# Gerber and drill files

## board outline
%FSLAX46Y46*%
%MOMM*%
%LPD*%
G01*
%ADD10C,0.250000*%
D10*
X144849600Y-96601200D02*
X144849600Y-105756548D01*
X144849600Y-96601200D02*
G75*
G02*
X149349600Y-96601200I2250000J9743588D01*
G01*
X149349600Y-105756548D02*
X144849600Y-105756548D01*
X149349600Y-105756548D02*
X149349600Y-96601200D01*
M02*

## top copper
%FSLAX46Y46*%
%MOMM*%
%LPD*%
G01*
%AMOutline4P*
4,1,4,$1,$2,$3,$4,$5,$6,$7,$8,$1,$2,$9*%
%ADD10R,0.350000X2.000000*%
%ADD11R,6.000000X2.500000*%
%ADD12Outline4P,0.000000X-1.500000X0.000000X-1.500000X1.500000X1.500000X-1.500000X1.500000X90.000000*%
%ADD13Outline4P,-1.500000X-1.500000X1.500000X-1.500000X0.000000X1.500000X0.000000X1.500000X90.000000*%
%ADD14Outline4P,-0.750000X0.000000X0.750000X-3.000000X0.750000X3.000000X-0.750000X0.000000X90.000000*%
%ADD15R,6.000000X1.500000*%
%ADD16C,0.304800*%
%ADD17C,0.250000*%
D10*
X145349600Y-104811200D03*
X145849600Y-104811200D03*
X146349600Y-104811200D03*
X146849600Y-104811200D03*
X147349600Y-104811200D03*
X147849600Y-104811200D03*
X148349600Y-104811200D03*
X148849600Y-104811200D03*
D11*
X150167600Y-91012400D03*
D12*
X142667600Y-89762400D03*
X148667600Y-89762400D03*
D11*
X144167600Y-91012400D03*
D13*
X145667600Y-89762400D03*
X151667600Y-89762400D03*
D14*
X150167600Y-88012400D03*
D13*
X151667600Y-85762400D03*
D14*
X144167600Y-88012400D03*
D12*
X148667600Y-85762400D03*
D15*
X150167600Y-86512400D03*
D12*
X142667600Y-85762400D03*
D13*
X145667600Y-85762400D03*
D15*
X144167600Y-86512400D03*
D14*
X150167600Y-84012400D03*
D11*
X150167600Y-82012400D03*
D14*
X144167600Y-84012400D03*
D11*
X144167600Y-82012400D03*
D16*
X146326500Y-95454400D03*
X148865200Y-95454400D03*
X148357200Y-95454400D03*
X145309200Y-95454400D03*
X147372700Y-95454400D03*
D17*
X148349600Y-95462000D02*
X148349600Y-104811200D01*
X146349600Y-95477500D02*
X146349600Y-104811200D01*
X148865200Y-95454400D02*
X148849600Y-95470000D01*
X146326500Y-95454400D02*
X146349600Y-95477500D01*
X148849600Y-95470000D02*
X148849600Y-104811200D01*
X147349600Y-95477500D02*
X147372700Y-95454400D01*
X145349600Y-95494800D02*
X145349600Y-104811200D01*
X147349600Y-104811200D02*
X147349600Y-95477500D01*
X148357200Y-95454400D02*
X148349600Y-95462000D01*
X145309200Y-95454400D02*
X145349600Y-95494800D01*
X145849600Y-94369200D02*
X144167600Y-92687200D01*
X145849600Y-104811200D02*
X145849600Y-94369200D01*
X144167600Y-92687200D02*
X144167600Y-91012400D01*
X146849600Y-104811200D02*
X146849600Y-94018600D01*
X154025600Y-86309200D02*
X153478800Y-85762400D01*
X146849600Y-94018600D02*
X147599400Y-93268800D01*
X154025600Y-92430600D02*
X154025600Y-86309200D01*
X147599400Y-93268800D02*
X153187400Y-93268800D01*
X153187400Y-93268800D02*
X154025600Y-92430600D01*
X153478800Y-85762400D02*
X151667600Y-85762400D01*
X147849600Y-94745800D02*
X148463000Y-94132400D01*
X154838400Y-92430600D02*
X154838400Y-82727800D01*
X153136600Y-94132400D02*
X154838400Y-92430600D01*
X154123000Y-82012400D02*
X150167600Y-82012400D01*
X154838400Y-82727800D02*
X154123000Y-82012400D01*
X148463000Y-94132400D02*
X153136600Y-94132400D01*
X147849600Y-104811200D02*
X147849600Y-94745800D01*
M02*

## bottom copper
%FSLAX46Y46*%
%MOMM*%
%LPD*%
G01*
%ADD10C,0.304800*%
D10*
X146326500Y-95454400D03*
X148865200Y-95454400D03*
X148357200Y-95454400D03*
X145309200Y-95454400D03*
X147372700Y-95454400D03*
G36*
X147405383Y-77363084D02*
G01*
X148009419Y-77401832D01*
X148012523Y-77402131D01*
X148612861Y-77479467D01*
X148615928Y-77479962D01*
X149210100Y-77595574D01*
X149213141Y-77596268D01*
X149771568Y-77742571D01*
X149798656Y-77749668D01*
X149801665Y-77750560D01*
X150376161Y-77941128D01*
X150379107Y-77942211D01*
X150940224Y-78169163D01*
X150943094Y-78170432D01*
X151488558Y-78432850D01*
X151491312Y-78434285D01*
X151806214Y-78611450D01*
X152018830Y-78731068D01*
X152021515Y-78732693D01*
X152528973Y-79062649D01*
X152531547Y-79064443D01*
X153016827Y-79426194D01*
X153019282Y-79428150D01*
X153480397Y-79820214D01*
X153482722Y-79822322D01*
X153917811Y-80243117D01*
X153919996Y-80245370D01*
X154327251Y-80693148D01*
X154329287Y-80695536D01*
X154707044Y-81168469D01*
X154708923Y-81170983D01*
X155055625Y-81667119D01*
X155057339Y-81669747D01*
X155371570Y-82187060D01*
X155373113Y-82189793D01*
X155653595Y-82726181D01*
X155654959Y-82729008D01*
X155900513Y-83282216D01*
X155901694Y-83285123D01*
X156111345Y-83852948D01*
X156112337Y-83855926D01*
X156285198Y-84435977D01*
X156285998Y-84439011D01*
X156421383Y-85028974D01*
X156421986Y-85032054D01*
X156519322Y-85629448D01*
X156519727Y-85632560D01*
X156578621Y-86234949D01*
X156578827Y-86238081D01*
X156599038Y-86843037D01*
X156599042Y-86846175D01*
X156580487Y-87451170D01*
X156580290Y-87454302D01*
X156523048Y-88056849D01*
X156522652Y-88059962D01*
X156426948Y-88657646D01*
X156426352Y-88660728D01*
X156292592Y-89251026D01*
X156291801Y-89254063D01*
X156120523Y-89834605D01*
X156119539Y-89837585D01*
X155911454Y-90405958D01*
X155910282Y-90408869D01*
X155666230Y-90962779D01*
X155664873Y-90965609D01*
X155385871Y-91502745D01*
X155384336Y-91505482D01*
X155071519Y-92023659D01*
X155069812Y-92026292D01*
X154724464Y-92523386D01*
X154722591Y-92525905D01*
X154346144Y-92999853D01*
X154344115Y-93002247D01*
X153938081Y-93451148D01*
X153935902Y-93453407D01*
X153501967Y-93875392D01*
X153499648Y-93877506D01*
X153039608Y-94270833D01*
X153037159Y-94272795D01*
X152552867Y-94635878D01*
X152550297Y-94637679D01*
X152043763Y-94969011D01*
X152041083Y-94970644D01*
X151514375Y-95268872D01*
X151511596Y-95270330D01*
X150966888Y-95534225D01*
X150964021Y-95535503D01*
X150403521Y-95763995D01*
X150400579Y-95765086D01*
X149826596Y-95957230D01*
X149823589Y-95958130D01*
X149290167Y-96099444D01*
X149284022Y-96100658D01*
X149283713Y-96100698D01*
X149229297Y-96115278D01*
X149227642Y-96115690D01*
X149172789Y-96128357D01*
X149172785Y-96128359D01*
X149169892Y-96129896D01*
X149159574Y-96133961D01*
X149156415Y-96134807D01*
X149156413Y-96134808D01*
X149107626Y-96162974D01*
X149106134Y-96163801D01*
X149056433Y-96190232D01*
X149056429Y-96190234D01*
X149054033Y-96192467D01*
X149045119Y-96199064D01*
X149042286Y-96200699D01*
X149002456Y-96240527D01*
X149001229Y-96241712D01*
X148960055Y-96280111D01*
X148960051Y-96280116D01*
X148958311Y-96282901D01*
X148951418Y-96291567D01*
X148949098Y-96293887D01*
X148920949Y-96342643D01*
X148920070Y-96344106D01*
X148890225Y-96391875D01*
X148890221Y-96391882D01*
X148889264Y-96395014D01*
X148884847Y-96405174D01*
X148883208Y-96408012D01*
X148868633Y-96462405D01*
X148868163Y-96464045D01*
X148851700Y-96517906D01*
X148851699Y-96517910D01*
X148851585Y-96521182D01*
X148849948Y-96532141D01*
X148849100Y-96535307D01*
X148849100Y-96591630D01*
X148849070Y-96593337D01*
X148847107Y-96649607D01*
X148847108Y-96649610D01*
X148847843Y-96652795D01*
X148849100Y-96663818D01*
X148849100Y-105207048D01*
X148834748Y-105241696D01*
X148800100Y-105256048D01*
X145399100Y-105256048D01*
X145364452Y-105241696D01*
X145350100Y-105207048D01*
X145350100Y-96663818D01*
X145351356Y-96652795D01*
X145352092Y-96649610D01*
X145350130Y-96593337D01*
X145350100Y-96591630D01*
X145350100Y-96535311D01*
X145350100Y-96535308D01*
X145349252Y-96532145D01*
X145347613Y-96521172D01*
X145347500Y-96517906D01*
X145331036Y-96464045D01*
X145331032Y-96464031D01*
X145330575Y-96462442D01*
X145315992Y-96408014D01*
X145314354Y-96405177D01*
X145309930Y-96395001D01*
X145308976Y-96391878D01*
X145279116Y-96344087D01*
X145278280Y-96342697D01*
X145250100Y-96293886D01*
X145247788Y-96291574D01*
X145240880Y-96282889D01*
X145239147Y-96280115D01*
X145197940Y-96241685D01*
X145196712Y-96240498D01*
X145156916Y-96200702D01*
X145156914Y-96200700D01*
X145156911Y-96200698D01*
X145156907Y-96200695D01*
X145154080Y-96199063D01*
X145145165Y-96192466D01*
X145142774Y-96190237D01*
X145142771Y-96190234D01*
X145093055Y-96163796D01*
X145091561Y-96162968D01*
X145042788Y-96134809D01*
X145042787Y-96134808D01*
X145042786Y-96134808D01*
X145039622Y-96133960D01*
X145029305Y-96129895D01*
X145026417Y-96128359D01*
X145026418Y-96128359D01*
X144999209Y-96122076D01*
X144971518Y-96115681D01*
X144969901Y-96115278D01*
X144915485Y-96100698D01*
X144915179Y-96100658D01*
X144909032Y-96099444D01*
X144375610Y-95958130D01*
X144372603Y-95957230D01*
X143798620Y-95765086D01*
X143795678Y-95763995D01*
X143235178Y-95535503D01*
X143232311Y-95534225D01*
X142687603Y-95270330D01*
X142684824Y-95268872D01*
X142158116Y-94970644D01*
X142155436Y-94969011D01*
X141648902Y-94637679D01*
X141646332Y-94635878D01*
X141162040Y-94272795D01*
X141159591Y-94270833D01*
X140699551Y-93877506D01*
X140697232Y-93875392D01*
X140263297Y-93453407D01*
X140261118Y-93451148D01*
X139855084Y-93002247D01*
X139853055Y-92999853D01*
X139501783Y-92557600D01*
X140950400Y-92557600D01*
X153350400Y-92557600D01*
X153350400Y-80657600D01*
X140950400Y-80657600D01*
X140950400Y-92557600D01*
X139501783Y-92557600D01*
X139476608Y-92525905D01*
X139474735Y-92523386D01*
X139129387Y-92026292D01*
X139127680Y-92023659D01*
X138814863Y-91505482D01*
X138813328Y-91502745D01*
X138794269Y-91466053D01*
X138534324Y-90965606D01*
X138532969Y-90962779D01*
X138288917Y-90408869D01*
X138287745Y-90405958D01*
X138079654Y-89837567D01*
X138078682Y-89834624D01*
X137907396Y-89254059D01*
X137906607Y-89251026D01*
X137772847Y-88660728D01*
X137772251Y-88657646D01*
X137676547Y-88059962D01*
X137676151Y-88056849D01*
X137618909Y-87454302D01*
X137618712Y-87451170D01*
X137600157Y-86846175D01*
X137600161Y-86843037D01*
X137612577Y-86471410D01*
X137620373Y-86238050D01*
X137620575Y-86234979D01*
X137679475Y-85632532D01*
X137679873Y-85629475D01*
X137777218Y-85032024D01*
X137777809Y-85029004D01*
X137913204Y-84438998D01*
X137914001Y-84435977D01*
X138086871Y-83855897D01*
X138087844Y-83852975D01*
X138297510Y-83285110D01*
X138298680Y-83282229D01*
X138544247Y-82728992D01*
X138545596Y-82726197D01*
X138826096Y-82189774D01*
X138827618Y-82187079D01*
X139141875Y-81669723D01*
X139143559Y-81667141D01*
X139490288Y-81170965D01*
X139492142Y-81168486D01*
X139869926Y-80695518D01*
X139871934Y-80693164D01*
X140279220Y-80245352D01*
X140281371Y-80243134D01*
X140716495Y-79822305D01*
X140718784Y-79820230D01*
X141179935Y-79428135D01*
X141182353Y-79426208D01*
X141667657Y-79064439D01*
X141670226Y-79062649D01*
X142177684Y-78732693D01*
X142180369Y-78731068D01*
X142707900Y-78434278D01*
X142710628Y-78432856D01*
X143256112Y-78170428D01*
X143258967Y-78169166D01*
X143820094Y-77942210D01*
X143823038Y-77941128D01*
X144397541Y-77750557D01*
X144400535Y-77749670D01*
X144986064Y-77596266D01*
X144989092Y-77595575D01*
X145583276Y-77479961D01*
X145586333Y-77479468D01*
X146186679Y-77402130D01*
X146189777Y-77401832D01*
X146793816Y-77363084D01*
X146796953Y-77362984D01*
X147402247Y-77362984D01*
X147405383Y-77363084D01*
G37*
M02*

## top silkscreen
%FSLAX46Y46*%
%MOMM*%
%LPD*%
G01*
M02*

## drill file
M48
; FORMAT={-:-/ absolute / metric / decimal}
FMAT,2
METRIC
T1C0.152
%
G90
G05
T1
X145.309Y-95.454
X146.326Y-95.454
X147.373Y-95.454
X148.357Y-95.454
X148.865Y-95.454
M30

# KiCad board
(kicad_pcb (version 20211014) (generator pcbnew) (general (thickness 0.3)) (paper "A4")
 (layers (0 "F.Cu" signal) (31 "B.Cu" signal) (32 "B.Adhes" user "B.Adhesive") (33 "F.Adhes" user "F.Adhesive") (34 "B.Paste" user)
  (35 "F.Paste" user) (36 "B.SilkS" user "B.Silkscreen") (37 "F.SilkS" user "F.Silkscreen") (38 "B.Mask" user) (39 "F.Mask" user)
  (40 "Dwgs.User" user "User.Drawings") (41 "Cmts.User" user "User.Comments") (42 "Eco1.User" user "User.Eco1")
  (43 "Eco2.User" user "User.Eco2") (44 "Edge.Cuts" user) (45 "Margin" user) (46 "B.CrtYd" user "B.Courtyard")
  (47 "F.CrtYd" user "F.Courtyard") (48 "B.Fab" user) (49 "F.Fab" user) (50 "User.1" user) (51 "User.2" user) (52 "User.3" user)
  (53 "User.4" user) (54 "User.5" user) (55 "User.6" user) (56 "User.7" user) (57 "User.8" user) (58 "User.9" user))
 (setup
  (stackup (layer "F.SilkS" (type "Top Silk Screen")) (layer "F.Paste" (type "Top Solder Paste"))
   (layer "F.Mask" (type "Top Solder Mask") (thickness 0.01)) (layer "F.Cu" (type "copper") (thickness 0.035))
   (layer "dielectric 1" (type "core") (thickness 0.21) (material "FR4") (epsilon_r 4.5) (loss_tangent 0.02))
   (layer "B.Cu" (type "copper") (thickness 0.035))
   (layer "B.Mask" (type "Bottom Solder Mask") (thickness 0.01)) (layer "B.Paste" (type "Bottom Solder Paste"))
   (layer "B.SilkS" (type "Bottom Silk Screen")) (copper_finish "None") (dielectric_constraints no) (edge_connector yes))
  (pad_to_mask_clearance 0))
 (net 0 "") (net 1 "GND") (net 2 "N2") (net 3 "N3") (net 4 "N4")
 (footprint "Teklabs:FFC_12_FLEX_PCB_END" (layer "F.Cu") (at 148.0996 104.6112)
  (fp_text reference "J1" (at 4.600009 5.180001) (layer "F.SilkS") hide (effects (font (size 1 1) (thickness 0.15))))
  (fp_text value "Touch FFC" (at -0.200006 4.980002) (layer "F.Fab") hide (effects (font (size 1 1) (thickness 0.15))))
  (pad "1" smd rect (at -2.75 0.2 180) (size 0.35 2) (layers "F.Cu" "F.Paste" "F.Mask") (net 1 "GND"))
  (pad "2" smd rect (at -2.25 0.2 180) (size 0.35 2) (layers "F.Cu" "F.Paste" "F.Mask") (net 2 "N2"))
  (pad "3" smd rect (at -1.75 0.2 180) (size 0.35 2) (layers "F.Cu" "F.Paste" "F.Mask") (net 1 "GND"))
  (pad "4" smd rect (at -1.25 0.2 180) (size 0.35 2) (layers "F.Cu" "F.Paste" "F.Mask") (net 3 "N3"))
  (pad "5" smd rect (at -0.75 0.2 180) (size 0.35 2) (layers "F.Cu" "F.Paste" "F.Mask") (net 1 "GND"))
  (pad "6" smd rect (at -0.25 0.2 180) (size 0.35 2) (layers "F.Cu" "F.Paste" "F.Mask") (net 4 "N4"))
  (pad "7" smd rect (at 0.25 0.2 180) (size 0.35 2) (layers "F.Cu" "F.Paste" "F.Mask") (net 1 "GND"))
  (pad "8" smd rect (at 0.75 0.2 180) (size 0.35 2) (layers "F.Cu" "F.Paste" "F.Mask") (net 1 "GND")))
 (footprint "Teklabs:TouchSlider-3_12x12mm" (layer "F.Cu") (at 146.3276 87.3524)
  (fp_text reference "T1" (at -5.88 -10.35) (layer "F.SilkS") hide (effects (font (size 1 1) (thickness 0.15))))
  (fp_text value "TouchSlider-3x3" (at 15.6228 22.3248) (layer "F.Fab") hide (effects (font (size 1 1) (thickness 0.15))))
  (pad "1" smd rect (at 3.84 3.66 90) (size 2.5 6) (layers "F.Cu" "F.Mask") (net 2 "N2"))
  (pad "1" smd trapezoid (at -3.66 2.41 90) (size 1.5 3) (rect_delta 0 -1.5) (layers "F.Cu" "F.Mask") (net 2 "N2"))
  (pad "1" smd trapezoid (at 2.34 2.41 90) (size 1.5 3) (rect_delta 0 -1.5) (layers "F.Cu" "F.Mask") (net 2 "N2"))
  (pad "1" smd rect (at -2.16 3.66 90) (size 2.5 6) (layers "F.Cu" "F.Mask") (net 2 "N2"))
  (pad "1" smd trapezoid (at -0.66 2.41 90) (size 1.5 3) (rect_delta 0 1.5) (layers "F.Cu" "F.Mask") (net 2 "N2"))
  (pad "1" smd trapezoid (at 5.34 2.41 90) (size 1.5 3) (rect_delta 0 1.5) (layers "F.Cu" "F.Mask") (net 2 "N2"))
  (pad "2" smd trapezoid (at 3.84 0.66 90) (size 1.5 3) (rect_delta -3 0) (layers "F.Cu" "F.Mask") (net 3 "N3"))
  (pad "2" smd trapezoid (at 5.34 -1.59 90) (size 1.5 3) (rect_delta 0 1.5) (layers "F.Cu" "F.Mask") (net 3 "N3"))
  (pad "2" smd trapezoid (at -2.16 0.66 90) (size 1.5 3) (rect_delta -3 0) (layers "F.Cu" "F.Mask") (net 3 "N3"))
  (pad "2" smd trapezoid (at 2.34 -1.59 90) (size 1.5 3) (rect_delta 0 -1.5) (layers "F.Cu" "F.Mask") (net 3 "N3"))
  (pad "2" smd rect (at 3.84 -0.84 90) (size 1.5 6) (layers "F.Cu" "F.Mask") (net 3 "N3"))
  (pad "2" smd trapezoid (at -3.66 -1.59 90) (size 1.5 3) (rect_delta 0 -1.5) (layers "F.Cu" "F.Mask") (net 3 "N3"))
  (pad "2" smd trapezoid (at -0.66 -1.59 90) (size 1.5 3) (rect_delta 0 1.5) (layers "F.Cu" "F.Mask") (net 3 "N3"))
  (pad "2" smd rect (at -2.16 -0.84 90) (size 1.5 6) (layers "F.Cu" "F.Mask") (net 3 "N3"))
  (pad "3" smd trapezoid (at 3.84 -3.34 90) (size 1.5 3) (rect_delta -3 0) (layers "F.Cu" "F.Mask") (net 4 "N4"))
  (pad "3" smd rect (at 3.84 -5.34 90) (size 2.5 6) (layers "F.Cu" "F.Mask") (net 4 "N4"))
  (pad "3" smd trapezoid (at -2.16 -3.34 90) (size 1.5 3) (rect_delta -3 0) (layers "F.Cu" "F.Mask") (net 4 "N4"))
  (pad "3" smd rect (at -2.16 -5.34 90) (size 2.5 6) (layers "F.Cu" "F.Mask") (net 4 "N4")))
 (gr_line (start 144.8496 96.6012) (end 144.8496 105.756548) (layer "Edge.Cuts") (width 0.25))
 (gr_arc (start 144.8496 96.6012) (mid 147.0996 76.857612) (end 149.3496 96.6012) (layer "Edge.Cuts") (width 0.25))
 (gr_line (start 149.3496 105.756548) (end 144.8496 105.756548) (layer "Edge.Cuts") (width 0.25))
 (gr_line (start 149.3496 105.756548) (end 149.3496 96.6012) (layer "Edge.Cuts") (width 0.25))
 (segment (start 148.3496 95.462) (end 148.3496 104.8112) (width 0.25) (layer "F.Cu") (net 1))
 (segment (start 146.3496 95.4775) (end 146.3496 104.8112) (width 0.25) (layer "F.Cu") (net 1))
 (segment (start 148.8652 95.4544) (end 148.8496 95.47) (width 0.25) (layer "F.Cu") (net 1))
 (segment (start 146.3265 95.4544) (end 146.3496 95.4775) (width 0.25) (layer "F.Cu") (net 1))
 (segment (start 148.8496 95.47) (end 148.8496 104.8112) (width 0.25) (layer "F.Cu") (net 1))
 (segment (start 147.3496 95.4775) (end 147.3727 95.4544) (width 0.25) (layer "F.Cu") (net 1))
 (segment (start 145.3496 95.4948) (end 145.3496 104.8112) (width 0.25) (layer "F.Cu") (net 1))
 (segment (start 147.3496 104.8112) (end 147.3496 95.4775) (width 0.25) (layer "F.Cu") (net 1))
 (segment (start 148.3572 95.4544) (end 148.3496 95.462) (width 0.25) (layer "F.Cu") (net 1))
 (segment (start 145.3092 95.4544) (end 145.3496 95.4948) (width 0.25) (layer "F.Cu") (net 1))
 (via (at 146.3265 95.4544) (size 0.3048) (drill 0.1524) (layers "F.Cu" "B.Cu") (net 1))
 (via (at 148.8652 95.4544) (size 0.3048) (drill 0.1524) (layers "F.Cu" "B.Cu") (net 1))
 (via (at 148.3572 95.4544) (size 0.3048) (drill 0.1524) (layers "F.Cu" "B.Cu") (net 1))
 (via (at 145.3092 95.4544) (size 0.3048) (drill 0.1524) (layers "F.Cu" "B.Cu") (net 1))
 (via (at 147.3727 95.4544) (size 0.3048) (drill 0.1524) (layers "F.Cu" "B.Cu") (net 1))
 (segment (start 145.8496 94.3692) (end 144.1676 92.6872) (width 0.25) (layer "F.Cu") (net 2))
 (segment (start 145.8496 104.8112) (end 145.8496 94.3692) (width 0.25) (layer "F.Cu") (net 2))
 (segment (start 144.1676 92.6872) (end 144.1676 91.0124) (width 0.25) (layer "F.Cu") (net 2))
 (segment (start 146.8496 104.8112) (end 146.8496 94.0186) (width 0.25) (layer "F.Cu") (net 3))
 (segment (start 154.0256 86.3092) (end 153.4788 85.7624) (width 0.25) (layer "F.Cu") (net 3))
 (segment (start 146.8496 94.0186) (end 147.5994 93.2688) (width 0.25) (layer "F.Cu") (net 3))
 (segment (start 154.0256 92.4306) (end 154.0256 86.3092) (width 0.25) (layer "F.Cu") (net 3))
 (segment (start 147.5994 93.2688) (end 153.1874 93.2688) (width 0.25) (layer "F.Cu") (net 3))
 (segment (start 153.1874 93.2688) (end 154.0256 92.4306) (width 0.25) (layer "F.Cu") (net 3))
 (segment (start 153.4788 85.7624) (end 151.6676 85.7624) (width 0.25) (layer "F.Cu") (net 3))
 (segment (start 147.8496 94.7458) (end 148.463 94.1324) (width 0.25) (layer "F.Cu") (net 4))
 (segment (start 154.8384 92.4306) (end 154.8384 82.7278) (width 0.25) (layer "F.Cu") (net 4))
 (segment (start 153.1366 94.1324) (end 154.8384 92.4306) (width 0.25) (layer "F.Cu") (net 4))
 (segment (start 154.123 82.0124) (end 150.1676 82.0124) (width 0.25) (layer "F.Cu") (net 4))
 (segment (start 154.8384 82.7278) (end 154.123 82.0124) (width 0.25) (layer "F.Cu") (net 4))
 (segment (start 148.463 94.1324) (end 153.1366 94.1324) (width 0.25) (layer "F.Cu") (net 4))
 (segment (start 147.8496 104.8112) (end 147.8496 94.7458) (width 0.25) (layer "F.Cu") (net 4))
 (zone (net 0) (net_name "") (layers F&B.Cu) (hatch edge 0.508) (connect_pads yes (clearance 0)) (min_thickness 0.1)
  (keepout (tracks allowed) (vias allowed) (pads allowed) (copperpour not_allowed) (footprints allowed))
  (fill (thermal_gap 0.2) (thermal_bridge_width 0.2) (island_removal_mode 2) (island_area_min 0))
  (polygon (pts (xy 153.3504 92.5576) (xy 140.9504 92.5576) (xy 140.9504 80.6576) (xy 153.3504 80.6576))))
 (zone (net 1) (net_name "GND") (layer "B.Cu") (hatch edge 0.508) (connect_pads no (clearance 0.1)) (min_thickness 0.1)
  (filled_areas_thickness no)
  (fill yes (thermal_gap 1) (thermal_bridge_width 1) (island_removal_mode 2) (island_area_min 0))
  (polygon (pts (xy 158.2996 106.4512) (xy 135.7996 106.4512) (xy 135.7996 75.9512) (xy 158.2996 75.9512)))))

